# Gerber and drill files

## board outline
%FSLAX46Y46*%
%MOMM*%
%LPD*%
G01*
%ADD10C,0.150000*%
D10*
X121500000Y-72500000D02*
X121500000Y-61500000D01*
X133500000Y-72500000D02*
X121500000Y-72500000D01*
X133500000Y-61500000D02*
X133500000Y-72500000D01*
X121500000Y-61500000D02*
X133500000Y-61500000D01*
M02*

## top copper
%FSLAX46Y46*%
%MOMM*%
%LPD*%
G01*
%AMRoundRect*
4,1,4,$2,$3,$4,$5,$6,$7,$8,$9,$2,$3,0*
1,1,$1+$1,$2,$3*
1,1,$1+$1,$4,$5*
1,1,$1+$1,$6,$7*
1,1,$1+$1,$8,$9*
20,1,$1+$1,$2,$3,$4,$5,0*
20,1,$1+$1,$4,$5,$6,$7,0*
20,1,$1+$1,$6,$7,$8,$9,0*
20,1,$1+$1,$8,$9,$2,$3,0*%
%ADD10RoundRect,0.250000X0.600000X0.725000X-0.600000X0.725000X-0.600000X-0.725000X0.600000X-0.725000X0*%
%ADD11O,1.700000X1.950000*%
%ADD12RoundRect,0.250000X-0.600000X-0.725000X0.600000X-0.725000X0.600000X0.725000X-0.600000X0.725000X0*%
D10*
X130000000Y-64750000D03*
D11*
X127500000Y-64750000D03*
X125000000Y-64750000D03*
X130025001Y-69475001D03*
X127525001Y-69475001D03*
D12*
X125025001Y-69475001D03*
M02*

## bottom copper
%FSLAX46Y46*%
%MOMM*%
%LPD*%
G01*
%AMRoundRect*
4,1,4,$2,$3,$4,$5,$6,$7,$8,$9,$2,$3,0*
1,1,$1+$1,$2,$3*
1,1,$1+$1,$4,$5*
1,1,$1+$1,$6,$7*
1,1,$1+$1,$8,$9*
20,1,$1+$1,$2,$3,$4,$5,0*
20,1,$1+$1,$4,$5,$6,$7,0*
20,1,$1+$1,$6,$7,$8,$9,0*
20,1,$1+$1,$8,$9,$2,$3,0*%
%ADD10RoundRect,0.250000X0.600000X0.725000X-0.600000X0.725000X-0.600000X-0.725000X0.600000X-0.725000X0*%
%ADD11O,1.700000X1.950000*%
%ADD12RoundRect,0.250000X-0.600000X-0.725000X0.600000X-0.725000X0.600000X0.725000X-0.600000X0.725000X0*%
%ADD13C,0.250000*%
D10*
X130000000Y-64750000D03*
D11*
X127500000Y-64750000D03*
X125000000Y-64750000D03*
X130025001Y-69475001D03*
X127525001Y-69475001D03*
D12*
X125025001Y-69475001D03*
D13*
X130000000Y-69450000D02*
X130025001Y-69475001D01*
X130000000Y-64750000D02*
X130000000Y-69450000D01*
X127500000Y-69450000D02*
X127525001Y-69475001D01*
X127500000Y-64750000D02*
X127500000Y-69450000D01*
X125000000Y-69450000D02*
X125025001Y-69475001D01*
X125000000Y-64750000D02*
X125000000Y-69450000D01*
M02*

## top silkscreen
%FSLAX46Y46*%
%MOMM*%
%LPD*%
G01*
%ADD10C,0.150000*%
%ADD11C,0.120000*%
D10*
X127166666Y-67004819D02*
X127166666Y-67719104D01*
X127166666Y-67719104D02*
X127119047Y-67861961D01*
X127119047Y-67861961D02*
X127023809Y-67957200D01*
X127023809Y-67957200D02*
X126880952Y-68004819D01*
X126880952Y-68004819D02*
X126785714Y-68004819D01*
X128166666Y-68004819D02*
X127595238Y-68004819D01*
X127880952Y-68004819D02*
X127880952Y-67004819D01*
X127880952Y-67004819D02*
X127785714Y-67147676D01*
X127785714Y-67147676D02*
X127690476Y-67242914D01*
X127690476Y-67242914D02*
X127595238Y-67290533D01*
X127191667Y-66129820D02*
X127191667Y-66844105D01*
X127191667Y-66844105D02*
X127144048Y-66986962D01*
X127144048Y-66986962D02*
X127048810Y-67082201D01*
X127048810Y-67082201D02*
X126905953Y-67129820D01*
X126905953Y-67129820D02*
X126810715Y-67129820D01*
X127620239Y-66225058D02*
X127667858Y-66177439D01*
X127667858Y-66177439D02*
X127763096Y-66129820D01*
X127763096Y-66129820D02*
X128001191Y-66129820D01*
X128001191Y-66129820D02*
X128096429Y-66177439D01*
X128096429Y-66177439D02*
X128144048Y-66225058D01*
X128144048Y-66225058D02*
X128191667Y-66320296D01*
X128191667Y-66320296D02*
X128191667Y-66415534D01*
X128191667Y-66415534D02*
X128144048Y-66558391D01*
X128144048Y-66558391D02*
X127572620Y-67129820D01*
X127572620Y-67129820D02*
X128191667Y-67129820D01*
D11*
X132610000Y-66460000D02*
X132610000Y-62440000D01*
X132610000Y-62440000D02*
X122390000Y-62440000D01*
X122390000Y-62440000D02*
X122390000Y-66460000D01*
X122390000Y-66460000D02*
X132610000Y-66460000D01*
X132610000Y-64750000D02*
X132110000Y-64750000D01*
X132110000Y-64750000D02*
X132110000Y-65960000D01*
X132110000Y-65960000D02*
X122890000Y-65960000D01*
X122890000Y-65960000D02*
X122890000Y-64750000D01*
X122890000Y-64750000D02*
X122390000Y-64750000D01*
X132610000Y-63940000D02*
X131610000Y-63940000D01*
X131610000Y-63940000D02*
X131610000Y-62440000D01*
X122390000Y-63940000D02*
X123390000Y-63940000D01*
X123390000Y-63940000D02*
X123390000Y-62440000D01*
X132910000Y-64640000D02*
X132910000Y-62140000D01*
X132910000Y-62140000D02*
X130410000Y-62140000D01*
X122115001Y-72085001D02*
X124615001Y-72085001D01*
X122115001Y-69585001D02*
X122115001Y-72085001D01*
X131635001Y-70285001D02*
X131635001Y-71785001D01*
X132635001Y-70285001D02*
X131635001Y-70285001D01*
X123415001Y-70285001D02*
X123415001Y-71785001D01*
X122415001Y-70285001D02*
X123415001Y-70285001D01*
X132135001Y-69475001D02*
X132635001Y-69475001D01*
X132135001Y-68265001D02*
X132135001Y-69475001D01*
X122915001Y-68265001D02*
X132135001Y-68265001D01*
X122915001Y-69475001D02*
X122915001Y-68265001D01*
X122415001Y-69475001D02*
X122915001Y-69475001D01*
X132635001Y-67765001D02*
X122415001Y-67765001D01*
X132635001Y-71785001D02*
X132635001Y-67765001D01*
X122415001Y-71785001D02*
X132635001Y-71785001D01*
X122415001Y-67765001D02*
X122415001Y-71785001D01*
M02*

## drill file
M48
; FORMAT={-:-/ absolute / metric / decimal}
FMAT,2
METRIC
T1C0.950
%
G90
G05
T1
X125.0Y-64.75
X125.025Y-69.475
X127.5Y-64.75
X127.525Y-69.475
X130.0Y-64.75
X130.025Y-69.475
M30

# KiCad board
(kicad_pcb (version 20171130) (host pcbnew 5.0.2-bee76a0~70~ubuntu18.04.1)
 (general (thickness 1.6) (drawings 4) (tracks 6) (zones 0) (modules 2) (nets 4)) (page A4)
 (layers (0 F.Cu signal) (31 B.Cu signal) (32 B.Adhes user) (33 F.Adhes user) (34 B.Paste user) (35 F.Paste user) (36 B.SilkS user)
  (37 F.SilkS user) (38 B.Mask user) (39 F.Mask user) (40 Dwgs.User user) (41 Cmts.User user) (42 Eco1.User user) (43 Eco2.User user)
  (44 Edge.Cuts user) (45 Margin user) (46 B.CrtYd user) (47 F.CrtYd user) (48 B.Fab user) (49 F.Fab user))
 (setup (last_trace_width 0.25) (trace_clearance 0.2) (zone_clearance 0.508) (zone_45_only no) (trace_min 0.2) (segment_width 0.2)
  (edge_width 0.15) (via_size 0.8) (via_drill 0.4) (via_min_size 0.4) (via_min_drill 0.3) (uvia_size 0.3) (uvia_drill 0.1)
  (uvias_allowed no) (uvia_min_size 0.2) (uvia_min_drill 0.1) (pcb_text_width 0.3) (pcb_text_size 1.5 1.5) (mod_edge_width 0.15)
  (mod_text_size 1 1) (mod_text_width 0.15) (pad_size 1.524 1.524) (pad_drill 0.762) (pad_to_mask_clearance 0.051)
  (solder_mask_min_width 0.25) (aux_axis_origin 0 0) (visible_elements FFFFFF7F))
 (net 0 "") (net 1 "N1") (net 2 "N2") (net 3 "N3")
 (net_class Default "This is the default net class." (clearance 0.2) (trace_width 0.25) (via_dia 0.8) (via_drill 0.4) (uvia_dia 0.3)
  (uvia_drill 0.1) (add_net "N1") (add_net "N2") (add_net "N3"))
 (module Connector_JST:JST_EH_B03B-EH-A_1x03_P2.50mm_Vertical (layer F.Cu) (at 130 64.75 180)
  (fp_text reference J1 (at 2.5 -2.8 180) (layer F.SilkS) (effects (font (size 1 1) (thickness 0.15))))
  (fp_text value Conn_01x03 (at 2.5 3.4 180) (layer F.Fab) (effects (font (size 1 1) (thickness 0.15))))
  (fp_line (start -2.61 -1.71) (end -2.61 2.31) (layer F.SilkS) (width 0.12))
  (fp_line (start -2.61 2.31) (end 7.61 2.31) (layer F.SilkS) (width 0.12))
  (fp_line (start 7.61 2.31) (end 7.61 -1.71) (layer F.SilkS) (width 0.12))
  (fp_line (start 7.61 -1.71) (end -2.61 -1.71) (layer F.SilkS) (width 0.12))
  (fp_line (start -2.61 0) (end -2.11 0) (layer F.SilkS) (width 0.12))
  (fp_line (start -2.11 0) (end -2.11 -1.21) (layer F.SilkS) (width 0.12))
  (fp_line (start -2.11 -1.21) (end 7.11 -1.21) (layer F.SilkS) (width 0.12))
  (fp_line (start 7.11 -1.21) (end 7.11 0) (layer F.SilkS) (width 0.12))
  (fp_line (start 7.11 0) (end 7.61 0) (layer F.SilkS) (width 0.12))
  (fp_line (start -2.61 0.81) (end -1.61 0.81) (layer F.SilkS) (width 0.12))
  (fp_line (start -1.61 0.81) (end -1.61 2.31) (layer F.SilkS) (width 0.12))
  (fp_line (start 7.61 0.81) (end 6.61 0.81) (layer F.SilkS) (width 0.12))
  (fp_line (start 6.61 0.81) (end 6.61 2.31) (layer F.SilkS) (width 0.12))
  (fp_line (start -2.91 0.11) (end -2.91 2.61) (layer F.SilkS) (width 0.12))
  (fp_line (start -2.91 2.61) (end -0.41 2.61) (layer F.SilkS) (width 0.12))
  (pad 1 thru_hole roundrect (at 0 0 180) (size 1.7 1.95) (drill 0.95) (layers *.Cu *.Mask) (roundrect_rratio 0.147059) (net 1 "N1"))
  (pad 2 thru_hole oval (at 2.5 0 180) (size 1.7 1.95) (drill 0.95) (layers *.Cu *.Mask) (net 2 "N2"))
  (pad 3 thru_hole oval (at 5 0 180) (size 1.7 1.95) (drill 0.95) (layers *.Cu *.Mask) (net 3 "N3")))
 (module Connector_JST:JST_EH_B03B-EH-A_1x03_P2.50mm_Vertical (layer F.Cu) (at 125.025001 69.475001)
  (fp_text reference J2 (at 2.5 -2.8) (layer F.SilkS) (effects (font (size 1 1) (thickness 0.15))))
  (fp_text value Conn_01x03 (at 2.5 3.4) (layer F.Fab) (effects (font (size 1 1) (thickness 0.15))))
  (fp_line (start -2.91 2.61) (end -0.41 2.61) (layer F.SilkS) (width 0.12))
  (fp_line (start -2.91 0.11) (end -2.91 2.61) (layer F.SilkS) (width 0.12))
  (fp_line (start 6.61 0.81) (end 6.61 2.31) (layer F.SilkS) (width 0.12))
  (fp_line (start 7.61 0.81) (end 6.61 0.81) (layer F.SilkS) (width 0.12))
  (fp_line (start -1.61 0.81) (end -1.61 2.31) (layer F.SilkS) (width 0.12))
  (fp_line (start -2.61 0.81) (end -1.61 0.81) (layer F.SilkS) (width 0.12))
  (fp_line (start 7.11 0) (end 7.61 0) (layer F.SilkS) (width 0.12))
  (fp_line (start 7.11 -1.21) (end 7.11 0) (layer F.SilkS) (width 0.12))
  (fp_line (start -2.11 -1.21) (end 7.11 -1.21) (layer F.SilkS) (width 0.12))
  (fp_line (start -2.11 0) (end -2.11 -1.21) (layer F.SilkS) (width 0.12))
  (fp_line (start -2.61 0) (end -2.11 0) (layer F.SilkS) (width 0.12))
  (fp_line (start 7.61 -1.71) (end -2.61 -1.71) (layer F.SilkS) (width 0.12))
  (fp_line (start 7.61 2.31) (end 7.61 -1.71) (layer F.SilkS) (width 0.12))
  (fp_line (start -2.61 2.31) (end 7.61 2.31) (layer F.SilkS) (width 0.12))
  (fp_line (start -2.61 -1.71) (end -2.61 2.31) (layer F.SilkS) (width 0.12))
  (pad 3 thru_hole oval (at 5 0) (size 1.7 1.95) (drill 0.95) (layers *.Cu *.Mask) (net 1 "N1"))
  (pad 2 thru_hole oval (at 2.5 0) (size 1.7 1.95) (drill 0.95) (layers *.Cu *.Mask) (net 2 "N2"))
  (pad 1 thru_hole roundrect (at 0 0) (size 1.7 1.95) (drill 0.95) (layers *.Cu *.Mask) (roundrect_rratio 0.147059) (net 3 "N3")))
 (gr_line (start 121.5 72.5) (end 121.5 61.5) (layer Edge.Cuts) (width 0.15))
 (gr_line (start 133.5 72.5) (end 121.5 72.5) (layer Edge.Cuts) (width 0.15))
 (gr_line (start 133.5 61.5) (end 133.5 72.5) (layer Edge.Cuts) (width 0.15))
 (gr_line (start 121.5 61.5) (end 133.5 61.5) (layer Edge.Cuts) (width 0.15))
 (segment (start 130 69.45) (end 130.025001 69.475001) (width 0.25) (layer B.Cu) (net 1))
 (segment (start 130 64.75) (end 130 69.45) (width 0.25) (layer B.Cu) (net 1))
 (segment (start 127.5 69.45) (end 127.525001 69.475001) (width 0.25) (layer B.Cu) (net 2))
 (segment (start 127.5 64.75) (end 127.5 69.45) (width 0.25) (layer B.Cu) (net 2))
 (segment (start 125 69.45) (end 125.025001 69.475001) (width 0.25) (layer B.Cu) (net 3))
 (segment (start 125 64.75) (end 125 69.45) (width 0.25) (layer B.Cu) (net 3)))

